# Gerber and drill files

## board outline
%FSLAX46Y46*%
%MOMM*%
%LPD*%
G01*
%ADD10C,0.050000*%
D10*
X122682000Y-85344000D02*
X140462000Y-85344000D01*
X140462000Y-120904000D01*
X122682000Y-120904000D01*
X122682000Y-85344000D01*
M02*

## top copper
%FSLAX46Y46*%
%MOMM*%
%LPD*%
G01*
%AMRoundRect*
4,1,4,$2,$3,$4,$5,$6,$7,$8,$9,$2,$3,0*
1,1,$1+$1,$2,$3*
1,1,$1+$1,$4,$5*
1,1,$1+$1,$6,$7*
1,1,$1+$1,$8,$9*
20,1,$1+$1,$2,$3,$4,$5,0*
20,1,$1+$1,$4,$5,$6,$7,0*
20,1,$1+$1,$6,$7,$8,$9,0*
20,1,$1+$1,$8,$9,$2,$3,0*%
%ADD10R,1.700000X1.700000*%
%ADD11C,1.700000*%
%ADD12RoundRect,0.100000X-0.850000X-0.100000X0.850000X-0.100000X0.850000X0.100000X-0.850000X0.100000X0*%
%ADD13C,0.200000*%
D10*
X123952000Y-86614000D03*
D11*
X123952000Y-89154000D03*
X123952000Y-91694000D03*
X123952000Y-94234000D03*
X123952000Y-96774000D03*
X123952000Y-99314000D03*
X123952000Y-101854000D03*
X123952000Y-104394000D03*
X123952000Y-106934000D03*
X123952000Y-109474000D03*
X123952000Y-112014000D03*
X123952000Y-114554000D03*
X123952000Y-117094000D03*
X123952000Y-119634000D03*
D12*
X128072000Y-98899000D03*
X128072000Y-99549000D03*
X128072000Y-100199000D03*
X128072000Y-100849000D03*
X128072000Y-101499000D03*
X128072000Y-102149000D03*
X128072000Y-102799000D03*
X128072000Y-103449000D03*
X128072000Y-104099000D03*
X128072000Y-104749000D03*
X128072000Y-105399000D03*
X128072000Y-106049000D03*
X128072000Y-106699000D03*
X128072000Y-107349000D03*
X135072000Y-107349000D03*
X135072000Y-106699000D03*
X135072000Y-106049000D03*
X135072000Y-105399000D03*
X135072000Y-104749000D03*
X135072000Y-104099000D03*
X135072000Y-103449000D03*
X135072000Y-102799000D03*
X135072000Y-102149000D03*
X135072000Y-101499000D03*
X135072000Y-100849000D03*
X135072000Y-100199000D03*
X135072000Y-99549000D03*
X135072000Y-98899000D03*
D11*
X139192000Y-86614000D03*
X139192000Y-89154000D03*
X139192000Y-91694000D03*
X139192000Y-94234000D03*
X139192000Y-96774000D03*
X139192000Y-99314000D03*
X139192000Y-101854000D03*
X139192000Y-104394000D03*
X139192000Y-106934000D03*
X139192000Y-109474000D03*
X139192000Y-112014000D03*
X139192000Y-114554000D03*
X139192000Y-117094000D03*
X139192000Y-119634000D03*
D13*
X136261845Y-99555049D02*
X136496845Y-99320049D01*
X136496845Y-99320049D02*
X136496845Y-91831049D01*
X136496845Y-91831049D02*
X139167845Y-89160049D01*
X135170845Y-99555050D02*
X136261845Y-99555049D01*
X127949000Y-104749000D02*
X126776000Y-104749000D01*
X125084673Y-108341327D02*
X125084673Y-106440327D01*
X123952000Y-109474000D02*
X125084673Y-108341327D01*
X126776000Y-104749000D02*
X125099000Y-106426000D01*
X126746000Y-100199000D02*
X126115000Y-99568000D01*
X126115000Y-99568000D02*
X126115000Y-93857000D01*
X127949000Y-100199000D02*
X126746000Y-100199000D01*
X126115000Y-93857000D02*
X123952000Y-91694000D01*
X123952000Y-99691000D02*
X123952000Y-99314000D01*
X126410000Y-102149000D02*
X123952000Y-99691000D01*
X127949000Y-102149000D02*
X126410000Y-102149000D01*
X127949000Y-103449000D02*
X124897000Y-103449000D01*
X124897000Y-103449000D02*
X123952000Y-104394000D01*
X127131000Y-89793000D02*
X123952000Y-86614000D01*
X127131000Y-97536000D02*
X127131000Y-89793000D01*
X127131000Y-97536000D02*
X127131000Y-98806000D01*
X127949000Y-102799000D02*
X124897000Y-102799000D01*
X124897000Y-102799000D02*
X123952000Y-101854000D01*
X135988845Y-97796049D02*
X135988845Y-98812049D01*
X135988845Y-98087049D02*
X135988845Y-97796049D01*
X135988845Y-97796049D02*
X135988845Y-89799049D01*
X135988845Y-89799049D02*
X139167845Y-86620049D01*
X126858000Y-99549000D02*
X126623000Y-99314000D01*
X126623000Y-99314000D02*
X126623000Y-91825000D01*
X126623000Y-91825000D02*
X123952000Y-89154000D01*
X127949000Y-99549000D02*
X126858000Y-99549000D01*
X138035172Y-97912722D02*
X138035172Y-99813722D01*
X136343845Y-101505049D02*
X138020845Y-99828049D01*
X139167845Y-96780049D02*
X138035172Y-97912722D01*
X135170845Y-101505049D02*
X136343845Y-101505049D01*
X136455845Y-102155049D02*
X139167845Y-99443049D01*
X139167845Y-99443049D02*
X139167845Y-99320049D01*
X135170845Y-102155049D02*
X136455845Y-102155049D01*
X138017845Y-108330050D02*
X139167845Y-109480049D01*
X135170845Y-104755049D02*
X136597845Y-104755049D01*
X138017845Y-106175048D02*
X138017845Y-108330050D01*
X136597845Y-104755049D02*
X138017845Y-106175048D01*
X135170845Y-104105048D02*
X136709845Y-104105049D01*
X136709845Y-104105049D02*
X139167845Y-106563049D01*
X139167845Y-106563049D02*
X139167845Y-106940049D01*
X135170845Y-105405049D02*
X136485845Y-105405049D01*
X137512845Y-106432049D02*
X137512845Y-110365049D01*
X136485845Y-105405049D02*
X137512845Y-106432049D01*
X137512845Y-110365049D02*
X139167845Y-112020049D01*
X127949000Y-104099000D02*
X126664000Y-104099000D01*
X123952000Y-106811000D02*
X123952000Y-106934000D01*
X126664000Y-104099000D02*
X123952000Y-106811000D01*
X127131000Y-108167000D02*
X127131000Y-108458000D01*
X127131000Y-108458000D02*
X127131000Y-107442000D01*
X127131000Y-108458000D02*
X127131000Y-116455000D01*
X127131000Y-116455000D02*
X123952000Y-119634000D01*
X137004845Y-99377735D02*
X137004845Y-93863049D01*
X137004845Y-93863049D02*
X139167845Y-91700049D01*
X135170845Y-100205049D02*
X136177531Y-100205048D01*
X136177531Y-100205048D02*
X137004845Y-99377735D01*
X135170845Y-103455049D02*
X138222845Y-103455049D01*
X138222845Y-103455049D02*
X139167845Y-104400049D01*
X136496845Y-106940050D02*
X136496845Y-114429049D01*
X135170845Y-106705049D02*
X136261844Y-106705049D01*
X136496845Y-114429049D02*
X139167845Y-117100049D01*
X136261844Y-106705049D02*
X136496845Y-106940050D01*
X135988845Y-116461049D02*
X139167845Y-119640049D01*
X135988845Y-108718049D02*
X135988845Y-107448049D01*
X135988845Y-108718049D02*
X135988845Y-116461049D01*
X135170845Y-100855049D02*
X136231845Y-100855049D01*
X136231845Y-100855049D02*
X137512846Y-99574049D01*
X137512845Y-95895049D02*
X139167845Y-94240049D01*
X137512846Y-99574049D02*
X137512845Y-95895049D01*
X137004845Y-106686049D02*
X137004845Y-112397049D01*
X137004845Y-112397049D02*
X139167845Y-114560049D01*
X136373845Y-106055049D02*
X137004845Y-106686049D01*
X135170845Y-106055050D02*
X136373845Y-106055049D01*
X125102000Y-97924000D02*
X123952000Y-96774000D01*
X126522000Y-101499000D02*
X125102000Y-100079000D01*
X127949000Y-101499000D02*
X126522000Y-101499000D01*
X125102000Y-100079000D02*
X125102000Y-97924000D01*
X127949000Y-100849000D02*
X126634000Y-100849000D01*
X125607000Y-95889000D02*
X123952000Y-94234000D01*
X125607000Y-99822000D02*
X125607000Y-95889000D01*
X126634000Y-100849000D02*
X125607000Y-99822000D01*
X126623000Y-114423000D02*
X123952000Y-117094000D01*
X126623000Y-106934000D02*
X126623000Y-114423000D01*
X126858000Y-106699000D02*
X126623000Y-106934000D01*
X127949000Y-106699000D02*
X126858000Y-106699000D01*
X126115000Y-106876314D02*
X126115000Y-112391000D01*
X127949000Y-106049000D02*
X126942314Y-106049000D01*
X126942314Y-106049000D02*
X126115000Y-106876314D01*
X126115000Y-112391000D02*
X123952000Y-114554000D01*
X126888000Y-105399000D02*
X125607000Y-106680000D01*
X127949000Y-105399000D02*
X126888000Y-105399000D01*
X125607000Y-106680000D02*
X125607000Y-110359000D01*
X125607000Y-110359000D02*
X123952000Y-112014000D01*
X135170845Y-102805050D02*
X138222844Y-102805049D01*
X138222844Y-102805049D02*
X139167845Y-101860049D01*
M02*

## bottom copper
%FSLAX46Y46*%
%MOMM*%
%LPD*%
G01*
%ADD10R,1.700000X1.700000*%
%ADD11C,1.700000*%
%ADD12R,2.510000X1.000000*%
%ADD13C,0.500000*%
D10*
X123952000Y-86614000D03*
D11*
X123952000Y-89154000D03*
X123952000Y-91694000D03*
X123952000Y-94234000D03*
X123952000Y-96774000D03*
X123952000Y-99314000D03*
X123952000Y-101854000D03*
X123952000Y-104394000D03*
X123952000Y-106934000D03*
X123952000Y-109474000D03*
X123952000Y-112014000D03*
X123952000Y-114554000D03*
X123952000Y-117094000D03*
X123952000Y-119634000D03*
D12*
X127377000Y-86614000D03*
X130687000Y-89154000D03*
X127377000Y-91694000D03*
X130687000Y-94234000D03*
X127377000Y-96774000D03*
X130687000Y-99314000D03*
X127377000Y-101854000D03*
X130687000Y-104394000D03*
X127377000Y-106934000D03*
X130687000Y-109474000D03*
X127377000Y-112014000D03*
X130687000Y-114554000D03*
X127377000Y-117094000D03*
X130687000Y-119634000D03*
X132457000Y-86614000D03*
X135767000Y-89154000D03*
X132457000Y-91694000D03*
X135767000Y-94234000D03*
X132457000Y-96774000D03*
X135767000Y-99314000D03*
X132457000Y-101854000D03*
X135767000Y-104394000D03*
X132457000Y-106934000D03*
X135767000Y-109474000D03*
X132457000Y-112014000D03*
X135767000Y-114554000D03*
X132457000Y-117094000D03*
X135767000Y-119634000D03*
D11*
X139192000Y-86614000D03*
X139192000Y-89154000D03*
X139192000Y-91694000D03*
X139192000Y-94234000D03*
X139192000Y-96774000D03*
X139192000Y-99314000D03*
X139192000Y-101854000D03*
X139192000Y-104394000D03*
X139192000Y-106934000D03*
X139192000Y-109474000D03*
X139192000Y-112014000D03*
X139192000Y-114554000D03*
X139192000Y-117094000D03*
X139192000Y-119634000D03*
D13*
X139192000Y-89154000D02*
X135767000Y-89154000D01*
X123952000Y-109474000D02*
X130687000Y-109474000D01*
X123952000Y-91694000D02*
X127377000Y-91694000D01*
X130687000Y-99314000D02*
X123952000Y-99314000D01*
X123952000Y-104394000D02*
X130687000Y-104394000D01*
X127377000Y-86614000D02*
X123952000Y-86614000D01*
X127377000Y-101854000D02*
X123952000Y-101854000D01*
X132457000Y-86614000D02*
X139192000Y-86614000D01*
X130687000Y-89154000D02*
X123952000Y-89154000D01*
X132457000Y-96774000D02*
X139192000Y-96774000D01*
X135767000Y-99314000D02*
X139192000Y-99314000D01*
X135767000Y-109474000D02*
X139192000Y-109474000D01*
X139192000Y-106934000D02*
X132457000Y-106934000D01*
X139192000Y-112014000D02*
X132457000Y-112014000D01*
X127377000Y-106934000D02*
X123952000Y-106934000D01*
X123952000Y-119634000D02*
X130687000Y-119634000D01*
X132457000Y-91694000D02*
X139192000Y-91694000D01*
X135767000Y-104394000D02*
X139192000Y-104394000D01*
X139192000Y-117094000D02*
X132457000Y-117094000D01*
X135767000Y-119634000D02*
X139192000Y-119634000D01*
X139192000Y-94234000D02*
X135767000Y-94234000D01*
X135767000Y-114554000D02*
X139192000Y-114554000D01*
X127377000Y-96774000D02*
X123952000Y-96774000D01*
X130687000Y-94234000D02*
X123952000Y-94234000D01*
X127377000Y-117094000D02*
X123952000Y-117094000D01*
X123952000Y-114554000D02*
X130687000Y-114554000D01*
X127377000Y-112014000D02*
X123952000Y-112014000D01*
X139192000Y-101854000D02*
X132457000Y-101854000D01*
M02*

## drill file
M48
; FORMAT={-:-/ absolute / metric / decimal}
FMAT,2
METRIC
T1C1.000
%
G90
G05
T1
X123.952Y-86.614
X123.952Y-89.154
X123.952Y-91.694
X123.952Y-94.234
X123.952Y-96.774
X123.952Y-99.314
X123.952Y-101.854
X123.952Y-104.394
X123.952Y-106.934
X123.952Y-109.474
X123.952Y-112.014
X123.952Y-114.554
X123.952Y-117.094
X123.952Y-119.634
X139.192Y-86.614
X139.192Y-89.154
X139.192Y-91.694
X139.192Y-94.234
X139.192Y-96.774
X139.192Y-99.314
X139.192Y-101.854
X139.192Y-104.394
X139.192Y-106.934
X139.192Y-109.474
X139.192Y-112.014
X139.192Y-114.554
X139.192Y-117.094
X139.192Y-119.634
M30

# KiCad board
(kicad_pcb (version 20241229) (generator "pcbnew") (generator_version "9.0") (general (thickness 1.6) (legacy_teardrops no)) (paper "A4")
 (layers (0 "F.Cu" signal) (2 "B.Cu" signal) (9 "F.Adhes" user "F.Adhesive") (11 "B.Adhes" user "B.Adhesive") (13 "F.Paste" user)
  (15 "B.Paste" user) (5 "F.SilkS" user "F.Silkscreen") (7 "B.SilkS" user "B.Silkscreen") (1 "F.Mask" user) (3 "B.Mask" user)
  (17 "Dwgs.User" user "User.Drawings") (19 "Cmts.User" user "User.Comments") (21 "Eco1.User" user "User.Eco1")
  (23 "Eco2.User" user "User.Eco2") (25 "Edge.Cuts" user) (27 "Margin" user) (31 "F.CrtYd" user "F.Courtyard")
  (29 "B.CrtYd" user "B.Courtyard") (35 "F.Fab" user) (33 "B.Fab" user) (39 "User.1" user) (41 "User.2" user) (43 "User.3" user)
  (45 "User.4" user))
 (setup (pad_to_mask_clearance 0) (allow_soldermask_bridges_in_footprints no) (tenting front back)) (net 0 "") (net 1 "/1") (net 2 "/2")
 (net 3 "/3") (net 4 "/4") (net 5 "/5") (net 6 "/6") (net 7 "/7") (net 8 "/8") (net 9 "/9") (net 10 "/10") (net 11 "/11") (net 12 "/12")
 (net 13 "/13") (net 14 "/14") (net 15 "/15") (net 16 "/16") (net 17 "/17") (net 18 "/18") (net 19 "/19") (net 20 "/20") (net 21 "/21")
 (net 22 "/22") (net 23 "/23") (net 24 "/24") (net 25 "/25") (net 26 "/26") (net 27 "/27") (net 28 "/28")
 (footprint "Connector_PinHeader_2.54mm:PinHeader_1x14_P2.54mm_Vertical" (layer "F.Cu") (at 123.952 86.614)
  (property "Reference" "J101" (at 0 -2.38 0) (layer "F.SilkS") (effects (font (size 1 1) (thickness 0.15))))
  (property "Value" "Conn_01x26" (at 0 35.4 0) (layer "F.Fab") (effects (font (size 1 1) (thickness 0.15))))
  (pad "1" thru_hole rect (at 0 0) (size 1.7 1.7) (drill 1) (layers "*.Cu" "*.Mask") (remove_unused_layers no) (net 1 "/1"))
  (pad "2" thru_hole circle (at 0 2.54) (size 1.7 1.7) (drill 1) (layers "*.Cu" "*.Mask") (remove_unused_layers no) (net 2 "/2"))
  (pad "3" thru_hole circle (at 0 5.08) (size 1.7 1.7) (drill 1) (layers "*.Cu" "*.Mask") (remove_unused_layers no) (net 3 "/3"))
  (pad "4" thru_hole circle (at 0 7.62) (size 1.7 1.7) (drill 1) (layers "*.Cu" "*.Mask") (remove_unused_layers no) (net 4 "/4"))
  (pad "5" thru_hole circle (at 0 10.16) (size 1.7 1.7) (drill 1) (layers "*.Cu" "*.Mask") (remove_unused_layers no) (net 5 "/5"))
  (pad "6" thru_hole circle (at 0 12.7) (size 1.7 1.7) (drill 1) (layers "*.Cu" "*.Mask") (remove_unused_layers no) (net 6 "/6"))
  (pad "7" thru_hole circle (at 0 15.24) (size 1.7 1.7) (drill 1) (layers "*.Cu" "*.Mask") (remove_unused_layers no) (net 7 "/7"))
  (pad "8" thru_hole circle (at 0 17.78) (size 1.7 1.7) (drill 1) (layers "*.Cu" "*.Mask") (remove_unused_layers no) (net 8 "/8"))
  (pad "9" thru_hole circle (at 0 20.32) (size 1.7 1.7) (drill 1) (layers "*.Cu" "*.Mask") (remove_unused_layers no) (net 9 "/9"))
  (pad "10" thru_hole circle (at 0 22.86) (size 1.7 1.7) (drill 1) (layers "*.Cu" "*.Mask") (remove_unused_layers no) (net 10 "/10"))
  (pad "11" thru_hole circle (at 0 25.4) (size 1.7 1.7) (drill 1) (layers "*.Cu" "*.Mask") (remove_unused_layers no) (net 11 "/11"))
  (pad "12" thru_hole circle (at 0 27.94) (size 1.7 1.7) (drill 1) (layers "*.Cu" "*.Mask") (remove_unused_layers no) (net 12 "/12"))
  (pad "13" thru_hole circle (at 0 30.48) (size 1.7 1.7) (drill 1) (layers "*.Cu" "*.Mask") (remove_unused_layers no) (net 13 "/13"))
  (pad "14" thru_hole circle (at 0 33.02) (size 1.7 1.7) (drill 1) (layers "*.Cu" "*.Mask") (remove_unused_layers no) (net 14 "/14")))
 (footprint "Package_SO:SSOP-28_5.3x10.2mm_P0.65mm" (layer "F.Cu") (at 131.572 103.124)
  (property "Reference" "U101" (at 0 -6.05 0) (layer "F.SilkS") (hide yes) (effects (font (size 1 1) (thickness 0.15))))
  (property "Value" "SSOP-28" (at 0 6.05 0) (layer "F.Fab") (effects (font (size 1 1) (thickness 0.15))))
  (pad "1" smd roundrect (at -3.5 -4.225) (size 1.9 0.4) (layers "F.Cu" "F.Mask" "F.Paste") (roundrect_rratio 0.25) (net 1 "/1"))
  (pad "2" smd roundrect (at -3.5 -3.575) (size 1.9 0.4) (layers "F.Cu" "F.Mask" "F.Paste") (roundrect_rratio 0.25) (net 2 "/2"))
  (pad "3" smd roundrect (at -3.5 -2.925) (size 1.9 0.4) (layers "F.Cu" "F.Mask" "F.Paste") (roundrect_rratio 0.25) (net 3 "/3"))
  (pad "4" smd roundrect (at -3.5 -2.275) (size 1.9 0.4) (layers "F.Cu" "F.Mask" "F.Paste") (roundrect_rratio 0.25) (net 4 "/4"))
  (pad "5" smd roundrect (at -3.5 -1.625) (size 1.9 0.4) (layers "F.Cu" "F.Mask" "F.Paste") (roundrect_rratio 0.25) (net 5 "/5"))
  (pad "6" smd roundrect (at -3.5 -0.975) (size 1.9 0.4) (layers "F.Cu" "F.Mask" "F.Paste") (roundrect_rratio 0.25) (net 6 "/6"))
  (pad "7" smd roundrect (at -3.5 -0.325) (size 1.9 0.4) (layers "F.Cu" "F.Mask" "F.Paste") (roundrect_rratio 0.25) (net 7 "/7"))
  (pad "8" smd roundrect (at -3.5 0.325) (size 1.9 0.4) (layers "F.Cu" "F.Mask" "F.Paste") (roundrect_rratio 0.25) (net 8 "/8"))
  (pad "9" smd roundrect (at -3.5 0.975) (size 1.9 0.4) (layers "F.Cu" "F.Mask" "F.Paste") (roundrect_rratio 0.25) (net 9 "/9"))
  (pad "10" smd roundrect (at -3.5 1.625) (size 1.9 0.4) (layers "F.Cu" "F.Mask" "F.Paste") (roundrect_rratio 0.25) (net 10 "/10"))
  (pad "11" smd roundrect (at -3.5 2.275) (size 1.9 0.4) (layers "F.Cu" "F.Mask" "F.Paste") (roundrect_rratio 0.25) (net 11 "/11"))
  (pad "12" smd roundrect (at -3.5 2.925) (size 1.9 0.4) (layers "F.Cu" "F.Mask" "F.Paste") (roundrect_rratio 0.25) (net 12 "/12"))
  (pad "13" smd roundrect (at -3.5 3.575) (size 1.9 0.4) (layers "F.Cu" "F.Mask" "F.Paste") (roundrect_rratio 0.25) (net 13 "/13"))
  (pad "14" smd roundrect (at -3.5 4.225) (size 1.9 0.4) (layers "F.Cu" "F.Mask" "F.Paste") (roundrect_rratio 0.25) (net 14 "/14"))
  (pad "15" smd roundrect (at 3.5 4.225) (size 1.9 0.4) (layers "F.Cu" "F.Mask" "F.Paste") (roundrect_rratio 0.25) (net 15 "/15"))
  (pad "16" smd roundrect (at 3.5 3.575) (size 1.9 0.4) (layers "F.Cu" "F.Mask" "F.Paste") (roundrect_rratio 0.25) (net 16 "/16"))
  (pad "17" smd roundrect (at 3.5 2.925) (size 1.9 0.4) (layers "F.Cu" "F.Mask" "F.Paste") (roundrect_rratio 0.25) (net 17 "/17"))
  (pad "18" smd roundrect (at 3.5 2.275) (size 1.9 0.4) (layers "F.Cu" "F.Mask" "F.Paste") (roundrect_rratio 0.25) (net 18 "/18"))
  (pad "19" smd roundrect (at 3.5 1.625) (size 1.9 0.4) (layers "F.Cu" "F.Mask" "F.Paste") (roundrect_rratio 0.25) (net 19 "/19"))
  (pad "20" smd roundrect (at 3.5 0.975) (size 1.9 0.4) (layers "F.Cu" "F.Mask" "F.Paste") (roundrect_rratio 0.25) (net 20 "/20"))
  (pad "21" smd roundrect (at 3.5 0.325) (size 1.9 0.4) (layers "F.Cu" "F.Mask" "F.Paste") (roundrect_rratio 0.25) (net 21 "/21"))
  (pad "22" smd roundrect (at 3.5 -0.325) (size 1.9 0.4) (layers "F.Cu" "F.Mask" "F.Paste") (roundrect_rratio 0.25) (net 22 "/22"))
  (pad "23" smd roundrect (at 3.5 -0.975) (size 1.9 0.4) (layers "F.Cu" "F.Mask" "F.Paste") (roundrect_rratio 0.25) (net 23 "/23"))
  (pad "24" smd roundrect (at 3.5 -1.625) (size 1.9 0.4) (layers "F.Cu" "F.Mask" "F.Paste") (roundrect_rratio 0.25) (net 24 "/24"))
  (pad "25" smd roundrect (at 3.5 -2.275) (size 1.9 0.4) (layers "F.Cu" "F.Mask" "F.Paste") (roundrect_rratio 0.25) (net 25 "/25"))
  (pad "26" smd roundrect (at 3.5 -2.925) (size 1.9 0.4) (layers "F.Cu" "F.Mask" "F.Paste") (roundrect_rratio 0.25) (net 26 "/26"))
  (pad "27" smd roundrect (at 3.5 -3.575) (size 1.9 0.4) (layers "F.Cu" "F.Mask" "F.Paste") (roundrect_rratio 0.25) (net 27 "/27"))
  (pad "28" smd roundrect (at 3.5 -4.225) (size 1.9 0.4) (layers "F.Cu" "F.Mask" "F.Paste") (roundrect_rratio 0.25) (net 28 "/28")))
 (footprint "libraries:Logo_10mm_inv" (layer "F.Cu") (at 131.572 112.268)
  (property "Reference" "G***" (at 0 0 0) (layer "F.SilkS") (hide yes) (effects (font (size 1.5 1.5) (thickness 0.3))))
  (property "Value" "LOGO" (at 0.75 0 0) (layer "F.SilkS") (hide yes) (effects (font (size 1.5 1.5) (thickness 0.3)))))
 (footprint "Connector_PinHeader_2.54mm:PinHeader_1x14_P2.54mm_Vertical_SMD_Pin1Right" (layer "B.Cu") (at 129.032 103.124 180)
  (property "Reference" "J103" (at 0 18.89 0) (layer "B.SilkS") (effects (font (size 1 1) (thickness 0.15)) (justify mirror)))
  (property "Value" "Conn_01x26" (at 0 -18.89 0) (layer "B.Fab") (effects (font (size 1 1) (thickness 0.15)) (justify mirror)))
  (pad "1" smd rect (at 1.655 16.51 180) (size 2.51 1) (layers "B.Cu" "B.Mask" "B.Paste") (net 1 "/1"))
  (pad "2" smd rect (at -1.655 13.97 180) (size 2.51 1) (layers "B.Cu" "B.Mask" "B.Paste") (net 2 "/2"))
  (pad "3" smd rect (at 1.655 11.43 180) (size 2.51 1) (layers "B.Cu" "B.Mask" "B.Paste") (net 3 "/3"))
  (pad "4" smd rect (at -1.655 8.89 180) (size 2.51 1) (layers "B.Cu" "B.Mask" "B.Paste") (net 4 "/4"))
  (pad "5" smd rect (at 1.655 6.35 180) (size 2.51 1) (layers "B.Cu" "B.Mask" "B.Paste") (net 5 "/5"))
  (pad "6" smd rect (at -1.655 3.81 180) (size 2.51 1) (layers "B.Cu" "B.Mask" "B.Paste") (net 6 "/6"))
  (pad "7" smd rect (at 1.655 1.27 180) (size 2.51 1) (layers "B.Cu" "B.Mask" "B.Paste") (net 7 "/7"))
  (pad "8" smd rect (at -1.655 -1.27 180) (size 2.51 1) (layers "B.Cu" "B.Mask" "B.Paste") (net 8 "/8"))
  (pad "9" smd rect (at 1.655 -3.81 180) (size 2.51 1) (layers "B.Cu" "B.Mask" "B.Paste") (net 9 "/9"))
  (pad "10" smd rect (at -1.655 -6.35 180) (size 2.51 1) (layers "B.Cu" "B.Mask" "B.Paste") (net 10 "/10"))
  (pad "11" smd rect (at 1.655 -8.89 180) (size 2.51 1) (layers "B.Cu" "B.Mask" "B.Paste") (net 11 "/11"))
  (pad "12" smd rect (at -1.655 -11.43 180) (size 2.51 1) (layers "B.Cu" "B.Mask" "B.Paste") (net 12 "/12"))
  (pad "13" smd rect (at 1.655 -13.97 180) (size 2.51 1) (layers "B.Cu" "B.Mask" "B.Paste") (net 13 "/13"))
  (pad "14" smd rect (at -1.655 -16.51 180) (size 2.51 1) (layers "B.Cu" "B.Mask" "B.Paste") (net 14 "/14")))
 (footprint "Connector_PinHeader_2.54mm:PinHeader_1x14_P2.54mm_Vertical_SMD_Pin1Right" (layer "B.Cu") (at 134.112 103.124 180)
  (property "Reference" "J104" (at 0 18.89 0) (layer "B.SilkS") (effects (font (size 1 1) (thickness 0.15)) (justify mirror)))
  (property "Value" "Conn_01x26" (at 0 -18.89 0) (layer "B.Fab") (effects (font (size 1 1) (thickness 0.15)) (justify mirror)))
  (pad "1" smd rect (at 1.655 16.51 180) (size 2.51 1) (layers "B.Cu" "B.Mask" "B.Paste") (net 28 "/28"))
  (pad "2" smd rect (at -1.655 13.97 180) (size 2.51 1) (layers "B.Cu" "B.Mask" "B.Paste") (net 27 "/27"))
  (pad "3" smd rect (at 1.655 11.43 180) (size 2.51 1) (layers "B.Cu" "B.Mask" "B.Paste") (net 26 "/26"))
  (pad "4" smd rect (at -1.655 8.89 180) (size 2.51 1) (layers "B.Cu" "B.Mask" "B.Paste") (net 25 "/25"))
  (pad "5" smd rect (at 1.655 6.35 180) (size 2.51 1) (layers "B.Cu" "B.Mask" "B.Paste") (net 24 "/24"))
  (pad "6" smd rect (at -1.655 3.81 180) (size 2.51 1) (layers "B.Cu" "B.Mask" "B.Paste") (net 23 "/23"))
  (pad "7" smd rect (at 1.655 1.27 180) (size 2.51 1) (layers "B.Cu" "B.Mask" "B.Paste") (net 22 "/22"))
  (pad "8" smd rect (at -1.655 -1.27 180) (size 2.51 1) (layers "B.Cu" "B.Mask" "B.Paste") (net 21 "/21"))
  (pad "9" smd rect (at 1.655 -3.81 180) (size 2.51 1) (layers "B.Cu" "B.Mask" "B.Paste") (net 20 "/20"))
  (pad "10" smd rect (at -1.655 -6.35 180) (size 2.51 1) (layers "B.Cu" "B.Mask" "B.Paste") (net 19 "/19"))
  (pad "11" smd rect (at 1.655 -8.89 180) (size 2.51 1) (layers "B.Cu" "B.Mask" "B.Paste") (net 18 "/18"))
  (pad "12" smd rect (at -1.655 -11.43 180) (size 2.51 1) (layers "B.Cu" "B.Mask" "B.Paste") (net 17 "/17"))
  (pad "13" smd rect (at 1.655 -13.97 180) (size 2.51 1) (layers "B.Cu" "B.Mask" "B.Paste") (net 16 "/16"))
  (pad "14" smd rect (at -1.655 -16.51 180) (size 2.51 1) (layers "B.Cu" "B.Mask" "B.Paste") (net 15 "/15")))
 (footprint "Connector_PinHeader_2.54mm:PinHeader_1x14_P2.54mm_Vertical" (layer "B.Cu") (at 139.192 86.614 180)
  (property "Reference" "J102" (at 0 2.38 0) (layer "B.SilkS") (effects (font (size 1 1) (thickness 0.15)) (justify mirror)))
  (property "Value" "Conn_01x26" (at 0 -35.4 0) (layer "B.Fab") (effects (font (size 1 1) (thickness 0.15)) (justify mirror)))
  (pad "1" thru_hole circle (at 0 0 180) (size 1.7 1.7) (drill 1) (layers "*.Cu" "*.Mask") (remove_unused_layers no) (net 28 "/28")
   (thermal_bridge_angle 90))
  (pad "2" thru_hole circle (at 0 -2.54 180) (size 1.7 1.7) (drill 1) (layers "*.Cu" "*.Mask") (remove_unused_layers no) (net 27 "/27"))
  (pad "3" thru_hole circle (at 0 -5.08 180) (size 1.7 1.7) (drill 1) (layers "*.Cu" "*.Mask") (remove_unused_layers no) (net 26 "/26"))
  (pad "4" thru_hole circle (at 0 -7.62 180) (size 1.7 1.7) (drill 1) (layers "*.Cu" "*.Mask") (remove_unused_layers no) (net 25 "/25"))
  (pad "5" thru_hole circle (at 0 -10.16 180) (size 1.7 1.7) (drill 1) (layers "*.Cu" "*.Mask") (remove_unused_layers no) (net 24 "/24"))
  (pad "6" thru_hole circle (at 0 -12.7 180) (size 1.7 1.7) (drill 1) (layers "*.Cu" "*.Mask") (remove_unused_layers no) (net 23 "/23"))
  (pad "7" thru_hole circle (at 0 -15.24 180) (size 1.7 1.7) (drill 1) (layers "*.Cu" "*.Mask") (remove_unused_layers no) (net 22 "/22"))
  (pad "8" thru_hole circle (at 0 -17.78 180) (size 1.7 1.7) (drill 1) (layers "*.Cu" "*.Mask") (remove_unused_layers no) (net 21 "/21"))
  (pad "9" thru_hole circle (at 0 -20.32 180) (size 1.7 1.7) (drill 1) (layers "*.Cu" "*.Mask") (remove_unused_layers no) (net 20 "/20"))
  (pad "10" thru_hole circle (at 0 -22.86 180) (size 1.7 1.7) (drill 1) (layers "*.Cu" "*.Mask") (remove_unused_layers no) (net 19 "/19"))
  (pad "11" thru_hole circle (at 0 -25.4 180) (size 1.7 1.7) (drill 1) (layers "*.Cu" "*.Mask") (remove_unused_layers no) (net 18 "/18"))
  (pad "12" thru_hole circle (at 0 -27.94 180) (size 1.7 1.7) (drill 1) (layers "*.Cu" "*.Mask") (remove_unused_layers no) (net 17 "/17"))
  (pad "13" thru_hole circle (at 0 -30.48 180) (size 1.7 1.7) (drill 1) (layers "*.Cu" "*.Mask") (remove_unused_layers no) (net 16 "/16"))
  (pad "14" thru_hole circle (at 0 -33.02 180) (size 1.7 1.7) (drill 1) (layers "*.Cu" "*.Mask") (remove_unused_layers no) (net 15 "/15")))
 (gr_rect (start 122.682 85.344) (end 140.462 120.904) (stroke (width 0.05) (type default)) (fill no) (layer "Edge.Cuts"))
 (segment (start 136.261845 99.555049) (end 136.496845 99.320049) (width 0.2) (layer "F.Cu") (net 27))
 (segment (start 136.496845 99.320049) (end 136.496845 91.831049) (width 0.2) (layer "F.Cu") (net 27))
 (segment (start 136.496845 91.831049) (end 139.167845 89.160049) (width 0.2) (layer "F.Cu") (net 27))
 (segment (start 135.170845 99.55505) (end 136.261845 99.555049) (width 0.2) (layer "F.Cu") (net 27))
 (segment (start 139.192 89.154) (end 135.767 89.154) (width 0.5) (layer "B.Cu") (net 27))
 (segment (start 127.949 104.749) (end 126.776 104.749) (width 0.2) (layer "F.Cu") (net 10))
 (segment (start 125.084673 108.341327) (end 125.084673 106.440327) (width 0.2) (layer "F.Cu") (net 10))
 (segment (start 123.952 109.474) (end 125.084673 108.341327) (width 0.2) (layer "F.Cu") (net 10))
 (segment (start 126.776 104.749) (end 125.099 106.426) (width 0.2) (layer "F.Cu") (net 10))
 (segment (start 123.952 109.474) (end 130.687 109.474) (width 0.5) (layer "B.Cu") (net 10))
 (segment (start 126.746 100.199) (end 126.115 99.568) (width 0.2) (layer "F.Cu") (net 3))
 (segment (start 126.115 99.568) (end 126.115 93.857) (width 0.2) (layer "F.Cu") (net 3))
 (segment (start 127.949 100.199) (end 126.746 100.199) (width 0.2) (layer "F.Cu") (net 3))
 (segment (start 126.115 93.857) (end 123.952 91.694) (width 0.2) (layer "F.Cu") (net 3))
 (segment (start 123.952 91.694) (end 127.377 91.694) (width 0.5) (layer "B.Cu") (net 3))
 (segment (start 123.952 99.691) (end 123.952 99.314) (width 0.2) (layer "F.Cu") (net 6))
 (segment (start 126.41 102.149) (end 123.952 99.691) (width 0.2) (layer "F.Cu") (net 6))
 (segment (start 127.949 102.149) (end 126.41 102.149) (width 0.2) (layer "F.Cu") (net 6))
 (segment (start 130.687 99.314) (end 123.952 99.314) (width 0.5) (layer "B.Cu") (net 6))
 (segment (start 127.949 103.449) (end 124.897 103.449) (width 0.2) (layer "F.Cu") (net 8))
 (segment (start 124.897 103.449) (end 123.952 104.394) (width 0.2) (layer "F.Cu") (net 8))
 (segment (start 123.952 104.394) (end 130.687 104.394) (width 0.5) (layer "B.Cu") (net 8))
 (segment (start 127.131 89.793) (end 123.952 86.614) (width 0.2) (layer "F.Cu") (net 1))
 (segment (start 127.131 97.536) (end 127.131 89.793) (width 0.2) (layer "F.Cu") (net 1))
 (segment (start 127.131 97.536) (end 127.131 98.806) (width 0.2) (layer "F.Cu") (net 1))
 (segment (start 127.377 86.614) (end 123.952 86.614) (width 0.5) (layer "B.Cu") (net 1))
 (segment (start 127.949 102.799) (end 124.897 102.799) (width 0.2) (layer "F.Cu") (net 7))
 (segment (start 124.897 102.799) (end 123.952 101.854) (width 0.2) (layer "F.Cu") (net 7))
 (segment (start 127.377 101.854) (end 123.952 101.854) (width 0.5) (layer "B.Cu") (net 7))
 (segment (start 135.988845 97.796049) (end 135.988845 98.812049) (width 0.2) (layer "F.Cu") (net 28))
 (segment (start 135.988845 98.087049) (end 135.988845 97.796049) (width 0.2) (layer "F.Cu") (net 28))
 (segment (start 135.988845 97.796049) (end 135.988845 89.799049) (width 0.2) (layer "F.Cu") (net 28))
 (segment (start 135.988845 89.799049) (end 139.167845 86.620049) (width 0.2) (layer "F.Cu") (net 28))
 (segment (start 132.457 86.614) (end 139.192 86.614) (width 0.5) (layer "B.Cu") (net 28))
 (segment (start 126.858 99.549) (end 126.623 99.314) (width 0.2) (layer "F.Cu") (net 2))
 (segment (start 126.623 99.314) (end 126.623 91.825) (width 0.2) (layer "F.Cu") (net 2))
 (segment (start 126.623 91.825) (end 123.952 89.154) (width 0.2) (layer "F.Cu") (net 2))
 (segment (start 127.949 99.549) (end 126.858 99.549) (width 0.2) (layer "F.Cu") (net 2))
 (segment (start 130.687 89.154) (end 123.952 89.154) (width 0.5) (layer "B.Cu") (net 2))
 (segment (start 138.035172 97.912722) (end 138.035172 99.813722) (width 0.2) (layer "F.Cu") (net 24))
 (segment (start 136.343845 101.505049) (end 138.020845 99.828049) (width 0.2) (layer "F.Cu") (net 24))
 (segment (start 139.167845 96.780049) (end 138.035172 97.912722) (width 0.2) (layer "F.Cu") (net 24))
 (segment (start 135.170845 101.505049) (end 136.343845 101.505049) (width 0.2) (layer "F.Cu") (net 24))
 (segment (start 132.457 96.774) (end 139.192 96.774) (width 0.5) (layer "B.Cu") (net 24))
 (segment (start 136.455845 102.155049) (end 139.167845 99.443049) (width 0.2) (layer "F.Cu") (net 23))
 (segment (start 139.167845 99.443049) (end 139.167845 99.320049) (width 0.2) (layer "F.Cu") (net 23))
 (segment (start 135.170845 102.155049) (end 136.455845 102.155049) (width 0.2) (layer "F.Cu") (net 23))
 (segment (start 135.767 99.314) (end 139.192 99.314) (width 0.5) (layer "B.Cu") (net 23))
 (segment (start 138.017845 108.33005) (end 139.167845 109.480049) (width 0.2) (layer "F.Cu") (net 19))
 (segment (start 135.170845 104.755049) (end 136.597845 104.755049) (width 0.2) (layer "F.Cu") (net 19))
 (segment (start 138.017845 106.175048) (end 138.017845 108.33005) (width 0.2) (layer "F.Cu") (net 19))
 (segment (start 136.597845 104.755049) (end 138.017845 106.175048) (width 0.2) (layer "F.Cu") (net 19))
 (segment (start 135.767 109.474) (end 139.192 109.474) (width 0.5) (layer "B.Cu") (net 19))
 (segment (start 135.170845 104.105048) (end 136.709845 104.105049) (width 0.2) (layer "F.Cu") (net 20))
 (segment (start 136.709845 104.105049) (end 139.167845 106.563049) (width 0.2) (layer "F.Cu") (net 20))
 (segment (start 139.167845 106.563049) (end 139.167845 106.940049) (width 0.2) (layer "F.Cu") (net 20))
 (segment (start 139.192 106.934) (end 132.457 106.934) (width 0.5) (layer "B.Cu") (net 20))
 (segment (start 135.170845 105.405049) (end 136.485845 105.405049) (width 0.2) (layer "F.Cu") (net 18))
 (segment (start 137.512845 106.432049) (end 137.512845 110.365049) (width 0.2) (layer "F.Cu") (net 18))
 (segment (start 136.485845 105.405049) (end 137.512845 106.432049) (width 0.2) (layer "F.Cu") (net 18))
 (segment (start 137.512845 110.365049) (end 139.167845 112.020049) (width 0.2) (layer "F.Cu") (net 18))
 (segment (start 139.192 112.014) (end 132.457 112.014) (width 0.5) (layer "B.Cu") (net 18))
 (segment (start 127.949 104.099) (end 126.664 104.099) (width 0.2) (layer "F.Cu") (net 9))
 (segment (start 123.952 106.811) (end 123.952 106.934) (width 0.2) (layer "F.Cu") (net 9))
 (segment (start 126.664 104.099) (end 123.952 106.811) (width 0.2) (layer "F.Cu") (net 9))
 (segment (start 127.377 106.934) (end 123.952 106.934) (width 0.5) (layer "B.Cu") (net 9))
 (segment (start 127.131 108.167) (end 127.131 108.458) (width 0.2) (layer "F.Cu") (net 14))
 (segment (start 127.131 108.458) (end 127.131 107.442) (width 0.2) (layer "F.Cu") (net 14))
 (segment (start 127.131 108.458) (end 127.131 116.455) (width 0.2) (layer "F.Cu") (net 14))
 (segment (start 127.131 116.455) (end 123.952 119.634) (width 0.2) (layer "F.Cu") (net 14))
 (segment (start 123.952 119.634) (end 130.687 119.634) (width 0.5) (layer "B.Cu") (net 14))
 (segment (start 137.004845 99.377735) (end 137.004845 93.863049) (width 0.2) (layer "F.Cu") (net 26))
 (segment (start 137.004845 93.863049) (end 139.167845 91.700049) (width 0.2) (layer "F.Cu") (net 26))
 (segment (start 135.170845 100.205049) (end 136.177531 100.205048) (width 0.2) (layer "F.Cu") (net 26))
 (segment (start 136.177531 100.205048) (end 137.004845 99.377735) (width 0.2) (layer "F.Cu") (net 26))
 (segment (start 132.457 91.694) (end 139.192 91.694) (width 0.5) (layer "B.Cu") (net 26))
 (segment (start 135.170845 103.455049) (end 138.222845 103.455049) (width 0.2) (layer "F.Cu") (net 21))
 (segment (start 138.222845 103.455049) (end 139.167845 104.400049) (width 0.2) (layer "F.Cu") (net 21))
 (segment (start 135.767 104.394) (end 139.192 104.394) (width 0.5) (layer "B.Cu") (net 21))
 (segment (start 136.496845 106.94005) (end 136.496845 114.429049) (width 0.2) (layer "F.Cu") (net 16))
 (segment (start 135.170845 106.705049) (end 136.261844 106.705049) (width 0.2) (layer "F.Cu") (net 16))
 (segment (start 136.496845 114.429049) (end 139.167845 117.100049) (width 0.2) (layer "F.Cu") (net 16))
 (segment (start 136.261844 106.705049) (end 136.496845 106.94005) (width 0.2) (layer "F.Cu") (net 16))
 (segment (start 139.192 117.094) (end 132.457 117.094) (width 0.5) (layer "B.Cu") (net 16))
 (segment (start 135.988845 116.461049) (end 139.167845 119.640049) (width 0.2) (layer "F.Cu") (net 15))
 (segment (start 135.988845 108.718049) (end 135.988845 107.448049) (width 0.2) (layer "F.Cu") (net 15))
 (segment (start 135.988845 108.718049) (end 135.988845 116.461049) (width 0.2) (layer "F.Cu") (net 15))
 (segment (start 135.767 119.634) (end 139.192 119.634) (width 0.5) (layer "B.Cu") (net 15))
 (segment (start 135.170845 100.855049) (end 136.231845 100.855049) (width 0.2) (layer "F.Cu") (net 25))
 (segment (start 136.231845 100.855049) (end 137.512846 99.574049) (width 0.2) (layer "F.Cu") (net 25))
 (segment (start 137.512845 95.895049) (end 139.167845 94.240049) (width 0.2) (layer "F.Cu") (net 25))
 (segment (start 137.512846 99.574049) (end 137.512845 95.895049) (width 0.2) (layer "F.Cu") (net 25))
 (segment (start 139.192 94.234) (end 135.767 94.234) (width 0.5) (layer "B.Cu") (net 25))
 (segment (start 137.004845 106.686049) (end 137.004845 112.397049) (width 0.2) (layer "F.Cu") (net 17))
 (segment (start 137.004845 112.397049) (end 139.167845 114.560049) (width 0.2) (layer "F.Cu") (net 17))
 (segment (start 136.373845 106.055049) (end 137.004845 106.686049) (width 0.2) (layer "F.Cu") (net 17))
 (segment (start 135.170845 106.05505) (end 136.373845 106.055049) (width 0.2) (layer "F.Cu") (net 17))
 (segment (start 135.767 114.554) (end 139.192 114.554) (width 0.5) (layer "B.Cu") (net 17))
 (segment (start 125.102 97.924) (end 123.952 96.774) (width 0.2) (layer "F.Cu") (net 5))
 (segment (start 126.522 101.499) (end 125.102 100.079) (width 0.2) (layer "F.Cu") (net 5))
 (segment (start 127.949 101.499) (end 126.522 101.499) (width 0.2) (layer "F.Cu") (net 5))
 (segment (start 125.102 100.079) (end 125.102 97.924) (width 0.2) (layer "F.Cu") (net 5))
 (segment (start 127.377 96.774) (end 123.952 96.774) (width 0.5) (layer "B.Cu") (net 5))
 (segment (start 127.949 100.849) (end 126.634 100.849) (width 0.2) (layer "F.Cu") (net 4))
 (segment (start 125.607 95.889) (end 123.952 94.234) (width 0.2) (layer "F.Cu") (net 4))
 (segment (start 125.607 99.822) (end 125.607 95.889) (width 0.2) (layer "F.Cu") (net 4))
 (segment (start 126.634 100.849) (end 125.607 99.822) (width 0.2) (layer "F.Cu") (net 4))
 (segment (start 130.687 94.234) (end 123.952 94.234) (width 0.5) (layer "B.Cu") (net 4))
 (segment (start 126.623 114.423) (end 123.952 117.094) (width 0.2) (layer "F.Cu") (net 13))
 (segment (start 126.623 106.934) (end 126.623 114.423) (width 0.2) (layer "F.Cu") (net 13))
 (segment (start 126.858 106.699) (end 126.623 106.934) (width 0.2) (layer "F.Cu") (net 13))
 (segment (start 127.949 106.699) (end 126.858 106.699) (width 0.2) (layer "F.Cu") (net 13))
 (segment (start 127.377 117.094) (end 123.952 117.094) (width 0.5) (layer "B.Cu") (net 13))
 (segment (start 126.115 106.876314) (end 126.115 112.391) (width 0.2) (layer "F.Cu") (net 12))
 (segment (start 127.949 106.049) (end 126.942314 106.049) (width 0.2) (layer "F.Cu") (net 12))
 (segment (start 126.942314 106.049) (end 126.115 106.876314) (width 0.2) (layer "F.Cu") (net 12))
 (segment (start 126.115 112.391) (end 123.952 114.554) (width 0.2) (layer "F.Cu") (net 12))
 (segment (start 123.952 114.554) (end 130.687 114.554) (width 0.5) (layer "B.Cu") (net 12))
 (segment (start 126.888 105.399) (end 125.607 106.68) (width 0.2) (layer "F.Cu") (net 11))
 (segment (start 127.949 105.399) (end 126.888 105.399) (width 0.2) (layer "F.Cu") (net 11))
 (segment (start 125.607 106.68) (end 125.607 110.359) (width 0.2) (layer "F.Cu") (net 11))
 (segment (start 125.607 110.359) (end 123.952 112.014) (width 0.2) (layer "F.Cu") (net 11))
 (segment (start 127.377 112.014) (end 123.952 112.014) (width 0.5) (layer "B.Cu") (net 11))
 (segment (start 135.170845 102.80505) (end 138.222844 102.805049) (width 0.2) (layer "F.Cu") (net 22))
 (segment (start 138.222844 102.805049) (end 139.167845 101.860049) (width 0.2) (layer "F.Cu") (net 22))
 (segment (start 139.192 101.854) (end 132.457 101.854) (width 0.5) (layer "B.Cu") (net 22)))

